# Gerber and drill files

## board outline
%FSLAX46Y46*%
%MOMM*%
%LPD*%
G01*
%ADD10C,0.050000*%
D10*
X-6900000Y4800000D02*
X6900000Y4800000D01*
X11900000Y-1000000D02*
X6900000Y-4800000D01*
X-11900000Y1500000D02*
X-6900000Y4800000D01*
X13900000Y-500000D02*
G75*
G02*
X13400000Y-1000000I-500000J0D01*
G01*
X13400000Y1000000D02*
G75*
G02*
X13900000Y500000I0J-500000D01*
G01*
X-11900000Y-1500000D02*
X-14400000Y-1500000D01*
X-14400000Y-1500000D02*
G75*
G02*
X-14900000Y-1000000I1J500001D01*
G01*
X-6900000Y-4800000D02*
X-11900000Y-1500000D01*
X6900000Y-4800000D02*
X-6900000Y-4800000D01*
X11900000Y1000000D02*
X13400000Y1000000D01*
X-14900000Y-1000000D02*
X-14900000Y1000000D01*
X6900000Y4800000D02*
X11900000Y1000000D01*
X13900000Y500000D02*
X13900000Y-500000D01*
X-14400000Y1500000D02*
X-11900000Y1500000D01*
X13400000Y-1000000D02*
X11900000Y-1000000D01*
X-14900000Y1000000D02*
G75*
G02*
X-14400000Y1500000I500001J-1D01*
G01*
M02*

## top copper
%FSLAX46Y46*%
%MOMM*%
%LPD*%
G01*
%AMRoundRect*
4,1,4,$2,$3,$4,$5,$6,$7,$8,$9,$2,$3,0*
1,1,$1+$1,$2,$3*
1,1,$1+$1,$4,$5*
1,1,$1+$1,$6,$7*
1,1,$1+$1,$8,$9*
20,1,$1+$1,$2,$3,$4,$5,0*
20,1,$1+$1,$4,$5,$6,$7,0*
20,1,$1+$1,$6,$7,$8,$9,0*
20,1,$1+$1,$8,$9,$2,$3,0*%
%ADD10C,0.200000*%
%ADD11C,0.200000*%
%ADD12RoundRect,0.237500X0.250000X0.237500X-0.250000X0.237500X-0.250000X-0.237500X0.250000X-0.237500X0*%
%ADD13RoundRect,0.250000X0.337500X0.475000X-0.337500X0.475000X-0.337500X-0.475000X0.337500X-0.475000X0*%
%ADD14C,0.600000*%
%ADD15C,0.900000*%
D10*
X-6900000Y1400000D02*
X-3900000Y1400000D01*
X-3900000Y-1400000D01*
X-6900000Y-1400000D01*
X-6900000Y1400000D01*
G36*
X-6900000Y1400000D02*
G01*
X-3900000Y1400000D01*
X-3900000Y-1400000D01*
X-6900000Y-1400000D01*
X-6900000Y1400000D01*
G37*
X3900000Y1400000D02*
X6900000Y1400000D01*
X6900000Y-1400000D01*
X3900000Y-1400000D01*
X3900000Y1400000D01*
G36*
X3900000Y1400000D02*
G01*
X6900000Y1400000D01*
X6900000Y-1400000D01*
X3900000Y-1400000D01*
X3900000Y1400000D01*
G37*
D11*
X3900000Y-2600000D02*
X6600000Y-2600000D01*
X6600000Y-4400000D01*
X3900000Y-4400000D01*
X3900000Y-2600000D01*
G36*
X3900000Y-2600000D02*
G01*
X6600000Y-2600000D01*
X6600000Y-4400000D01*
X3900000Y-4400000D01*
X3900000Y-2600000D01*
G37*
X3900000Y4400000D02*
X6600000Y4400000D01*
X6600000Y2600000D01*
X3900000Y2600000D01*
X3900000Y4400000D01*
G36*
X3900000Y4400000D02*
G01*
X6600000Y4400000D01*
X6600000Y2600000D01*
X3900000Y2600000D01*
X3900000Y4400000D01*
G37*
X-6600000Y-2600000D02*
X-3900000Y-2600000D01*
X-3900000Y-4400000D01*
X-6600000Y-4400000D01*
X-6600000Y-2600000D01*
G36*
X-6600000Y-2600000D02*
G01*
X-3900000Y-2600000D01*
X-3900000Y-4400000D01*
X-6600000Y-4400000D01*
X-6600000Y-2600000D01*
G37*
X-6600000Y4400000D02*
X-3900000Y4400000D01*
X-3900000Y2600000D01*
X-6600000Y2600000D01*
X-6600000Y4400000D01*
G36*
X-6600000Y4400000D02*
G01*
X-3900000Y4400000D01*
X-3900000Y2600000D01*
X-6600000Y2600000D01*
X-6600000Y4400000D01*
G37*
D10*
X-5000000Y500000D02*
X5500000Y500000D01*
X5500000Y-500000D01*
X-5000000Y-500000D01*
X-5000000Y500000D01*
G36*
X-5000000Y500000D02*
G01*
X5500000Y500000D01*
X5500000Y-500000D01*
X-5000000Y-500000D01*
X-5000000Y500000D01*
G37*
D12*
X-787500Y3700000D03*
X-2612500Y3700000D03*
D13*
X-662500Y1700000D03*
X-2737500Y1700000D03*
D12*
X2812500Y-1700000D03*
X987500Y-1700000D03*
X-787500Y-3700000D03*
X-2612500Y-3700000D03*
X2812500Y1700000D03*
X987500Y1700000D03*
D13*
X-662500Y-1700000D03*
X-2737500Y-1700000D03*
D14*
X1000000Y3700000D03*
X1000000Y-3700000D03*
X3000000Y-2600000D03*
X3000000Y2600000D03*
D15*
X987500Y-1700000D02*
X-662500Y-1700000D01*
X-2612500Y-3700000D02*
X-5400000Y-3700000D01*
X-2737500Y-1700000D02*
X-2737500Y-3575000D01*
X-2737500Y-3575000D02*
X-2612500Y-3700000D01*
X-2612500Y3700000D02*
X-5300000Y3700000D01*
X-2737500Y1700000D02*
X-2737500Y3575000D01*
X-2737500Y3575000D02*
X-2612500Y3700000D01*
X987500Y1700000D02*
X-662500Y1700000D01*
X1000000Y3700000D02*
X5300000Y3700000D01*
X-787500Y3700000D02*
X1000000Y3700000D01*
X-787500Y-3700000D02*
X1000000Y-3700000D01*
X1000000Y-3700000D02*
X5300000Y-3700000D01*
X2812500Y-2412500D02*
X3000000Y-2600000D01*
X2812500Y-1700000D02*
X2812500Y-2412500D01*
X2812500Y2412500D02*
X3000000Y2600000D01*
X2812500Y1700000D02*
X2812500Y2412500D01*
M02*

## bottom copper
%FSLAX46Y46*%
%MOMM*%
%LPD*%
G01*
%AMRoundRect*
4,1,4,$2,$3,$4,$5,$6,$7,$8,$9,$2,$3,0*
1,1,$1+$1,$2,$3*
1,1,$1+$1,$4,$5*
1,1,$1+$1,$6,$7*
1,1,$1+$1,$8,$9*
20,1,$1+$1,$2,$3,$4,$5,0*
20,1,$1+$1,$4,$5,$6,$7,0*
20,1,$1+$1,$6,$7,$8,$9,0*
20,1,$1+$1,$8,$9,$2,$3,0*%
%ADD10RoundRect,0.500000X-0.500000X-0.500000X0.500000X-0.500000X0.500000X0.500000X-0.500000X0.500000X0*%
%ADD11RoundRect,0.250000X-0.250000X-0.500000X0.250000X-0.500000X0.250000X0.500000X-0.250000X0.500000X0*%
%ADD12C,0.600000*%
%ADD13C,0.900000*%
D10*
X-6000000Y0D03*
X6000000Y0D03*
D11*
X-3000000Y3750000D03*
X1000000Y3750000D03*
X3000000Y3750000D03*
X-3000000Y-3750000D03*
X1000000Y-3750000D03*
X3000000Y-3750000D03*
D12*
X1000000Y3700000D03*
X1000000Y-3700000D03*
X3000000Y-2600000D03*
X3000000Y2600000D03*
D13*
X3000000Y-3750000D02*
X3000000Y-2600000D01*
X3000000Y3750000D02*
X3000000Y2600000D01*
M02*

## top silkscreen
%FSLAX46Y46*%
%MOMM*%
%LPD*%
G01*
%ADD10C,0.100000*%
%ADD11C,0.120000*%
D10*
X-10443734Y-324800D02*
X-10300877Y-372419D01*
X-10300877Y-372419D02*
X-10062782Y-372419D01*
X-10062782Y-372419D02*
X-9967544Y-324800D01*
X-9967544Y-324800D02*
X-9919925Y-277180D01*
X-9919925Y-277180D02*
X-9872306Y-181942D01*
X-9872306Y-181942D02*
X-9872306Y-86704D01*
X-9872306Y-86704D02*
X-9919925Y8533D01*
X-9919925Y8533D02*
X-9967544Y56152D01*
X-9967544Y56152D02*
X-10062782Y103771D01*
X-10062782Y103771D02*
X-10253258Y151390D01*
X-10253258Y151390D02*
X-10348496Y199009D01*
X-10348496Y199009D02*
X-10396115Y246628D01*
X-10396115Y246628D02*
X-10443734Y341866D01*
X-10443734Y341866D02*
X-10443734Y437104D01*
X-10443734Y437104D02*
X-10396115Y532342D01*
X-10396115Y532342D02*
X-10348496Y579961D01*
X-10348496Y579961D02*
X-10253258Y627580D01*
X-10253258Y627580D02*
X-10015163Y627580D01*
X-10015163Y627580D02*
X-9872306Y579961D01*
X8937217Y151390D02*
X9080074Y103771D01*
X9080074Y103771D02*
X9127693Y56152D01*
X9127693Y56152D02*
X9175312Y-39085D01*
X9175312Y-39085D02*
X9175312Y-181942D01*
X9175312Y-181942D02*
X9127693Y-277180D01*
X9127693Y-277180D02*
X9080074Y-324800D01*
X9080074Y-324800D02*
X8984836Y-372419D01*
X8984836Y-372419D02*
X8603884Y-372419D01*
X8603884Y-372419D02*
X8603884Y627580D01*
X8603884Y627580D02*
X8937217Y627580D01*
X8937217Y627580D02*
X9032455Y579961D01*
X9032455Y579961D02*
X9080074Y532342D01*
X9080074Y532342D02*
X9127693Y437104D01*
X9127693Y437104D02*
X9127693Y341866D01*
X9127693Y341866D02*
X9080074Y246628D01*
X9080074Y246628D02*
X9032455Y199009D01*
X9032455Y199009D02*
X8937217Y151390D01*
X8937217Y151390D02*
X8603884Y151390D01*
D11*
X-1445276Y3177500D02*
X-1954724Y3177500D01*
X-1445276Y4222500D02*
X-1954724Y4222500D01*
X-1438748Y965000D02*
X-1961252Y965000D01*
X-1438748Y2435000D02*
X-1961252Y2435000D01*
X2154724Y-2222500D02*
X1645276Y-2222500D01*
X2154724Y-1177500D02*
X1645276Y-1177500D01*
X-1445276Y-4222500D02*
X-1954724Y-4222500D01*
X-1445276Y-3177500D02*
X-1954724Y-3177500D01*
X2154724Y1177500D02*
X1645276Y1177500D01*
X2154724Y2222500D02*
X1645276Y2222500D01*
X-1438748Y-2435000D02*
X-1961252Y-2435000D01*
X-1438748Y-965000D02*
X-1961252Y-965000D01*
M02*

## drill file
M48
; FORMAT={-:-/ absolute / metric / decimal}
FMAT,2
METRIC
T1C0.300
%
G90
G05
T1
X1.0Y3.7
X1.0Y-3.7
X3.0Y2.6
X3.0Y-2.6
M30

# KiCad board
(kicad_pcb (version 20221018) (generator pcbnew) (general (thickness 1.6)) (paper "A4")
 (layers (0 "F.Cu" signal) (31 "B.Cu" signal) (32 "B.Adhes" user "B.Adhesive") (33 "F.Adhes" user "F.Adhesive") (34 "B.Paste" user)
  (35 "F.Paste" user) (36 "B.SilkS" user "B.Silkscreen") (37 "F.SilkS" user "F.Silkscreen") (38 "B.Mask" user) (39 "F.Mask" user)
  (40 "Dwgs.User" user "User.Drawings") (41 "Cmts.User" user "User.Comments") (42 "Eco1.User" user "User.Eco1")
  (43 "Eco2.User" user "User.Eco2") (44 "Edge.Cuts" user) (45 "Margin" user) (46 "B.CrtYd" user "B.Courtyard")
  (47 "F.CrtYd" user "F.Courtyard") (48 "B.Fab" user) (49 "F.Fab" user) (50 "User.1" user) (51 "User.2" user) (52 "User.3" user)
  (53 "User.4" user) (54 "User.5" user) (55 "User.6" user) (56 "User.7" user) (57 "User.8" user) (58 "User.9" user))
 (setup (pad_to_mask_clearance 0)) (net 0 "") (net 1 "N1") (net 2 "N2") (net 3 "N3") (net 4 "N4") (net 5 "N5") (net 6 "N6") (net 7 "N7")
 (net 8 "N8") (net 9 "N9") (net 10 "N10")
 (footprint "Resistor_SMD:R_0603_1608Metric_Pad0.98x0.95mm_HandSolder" (layer "F.Cu") (at -1.7 -3.7 180)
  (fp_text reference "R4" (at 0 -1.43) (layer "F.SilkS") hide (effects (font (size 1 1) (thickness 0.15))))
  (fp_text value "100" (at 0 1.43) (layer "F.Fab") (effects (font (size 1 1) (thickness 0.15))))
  (fp_line (start -0.254724 -0.5225) (end 0.254724 -0.5225) (stroke (width 0.12) (type solid)) (layer "F.SilkS"))
  (fp_line (start -0.254724 0.5225) (end 0.254724 0.5225) (stroke (width 0.12) (type solid)) (layer "F.SilkS"))
  (pad "1" smd roundrect (at -0.9125 0 180) (size 0.975 0.95) (layers "F.Cu" "F.Paste" "F.Mask") (roundrect_rratio 0.25) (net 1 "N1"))
  (pad "2" smd roundrect (at 0.9125 0 180) (size 0.975 0.95) (layers "F.Cu" "F.Paste" "F.Mask") (roundrect_rratio 0.25) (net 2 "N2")))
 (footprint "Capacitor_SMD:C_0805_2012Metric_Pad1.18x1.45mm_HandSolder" (layer "F.Cu") (at -1.7 -1.7 180)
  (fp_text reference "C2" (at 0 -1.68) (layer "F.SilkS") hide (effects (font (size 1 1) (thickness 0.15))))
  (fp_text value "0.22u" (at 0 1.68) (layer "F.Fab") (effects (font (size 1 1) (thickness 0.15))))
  (fp_line (start -0.261252 -0.735) (end 0.261252 -0.735) (stroke (width 0.12) (type solid)) (layer "F.SilkS"))
  (fp_line (start -0.261252 0.735) (end 0.261252 0.735) (stroke (width 0.12) (type solid)) (layer "F.SilkS"))
  (pad "1" smd roundrect (at -1.0375 0 180) (size 1.175 1.45) (layers "F.Cu" "F.Paste" "F.Mask") (roundrect_rratio 0.2127659574)
   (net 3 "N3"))
  (pad "2" smd roundrect (at 1.0375 0 180) (size 1.175 1.45) (layers "F.Cu" "F.Paste" "F.Mask") (roundrect_rratio 0.2127659574) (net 2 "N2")))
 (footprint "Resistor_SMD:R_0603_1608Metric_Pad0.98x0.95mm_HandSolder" (layer "F.Cu") (at 1.9 1.7 180)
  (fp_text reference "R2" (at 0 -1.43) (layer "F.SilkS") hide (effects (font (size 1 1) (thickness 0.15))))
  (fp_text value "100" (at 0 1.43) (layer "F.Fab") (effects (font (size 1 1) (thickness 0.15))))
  (fp_line (start -0.254724 -0.5225) (end 0.254724 -0.5225) (stroke (width 0.12) (type solid)) (layer "F.SilkS"))
  (fp_line (start -0.254724 0.5225) (end 0.254724 0.5225) (stroke (width 0.12) (type solid)) (layer "F.SilkS"))
  (pad "1" smd roundrect (at -0.9125 0 180) (size 0.975 0.95) (layers "F.Cu" "F.Paste" "F.Mask") (roundrect_rratio 0.25) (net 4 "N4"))
  (pad "2" smd roundrect (at 0.9125 0 180) (size 0.975 0.95) (layers "F.Cu" "F.Paste" "F.Mask") (roundrect_rratio 0.25) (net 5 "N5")))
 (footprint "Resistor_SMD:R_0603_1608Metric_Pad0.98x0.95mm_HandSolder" (layer "F.Cu") (at -1.7 3.7 180)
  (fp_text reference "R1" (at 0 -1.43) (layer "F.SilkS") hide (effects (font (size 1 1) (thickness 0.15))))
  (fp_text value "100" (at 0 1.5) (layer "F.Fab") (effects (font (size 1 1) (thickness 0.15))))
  (fp_line (start -0.254724 -0.5225) (end 0.254724 -0.5225) (stroke (width 0.12) (type solid)) (layer "F.SilkS"))
  (fp_line (start -0.254724 0.5225) (end 0.254724 0.5225) (stroke (width 0.12) (type solid)) (layer "F.SilkS"))
  (pad "1" smd roundrect (at -0.9125 0 180) (size 0.975 0.95) (layers "F.Cu" "F.Paste" "F.Mask") (roundrect_rratio 0.25) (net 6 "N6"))
  (pad "2" smd roundrect (at 0.9125 0 180) (size 0.975 0.95) (layers "F.Cu" "F.Paste" "F.Mask") (roundrect_rratio 0.25) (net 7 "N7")))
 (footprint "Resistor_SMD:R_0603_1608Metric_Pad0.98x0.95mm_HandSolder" (layer "F.Cu") (at 1.9 -1.7 180)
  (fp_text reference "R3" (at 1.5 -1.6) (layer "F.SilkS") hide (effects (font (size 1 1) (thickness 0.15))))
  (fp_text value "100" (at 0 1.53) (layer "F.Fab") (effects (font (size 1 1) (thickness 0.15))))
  (fp_line (start -0.254724 -0.5225) (end 0.254724 -0.5225) (stroke (width 0.12) (type solid)) (layer "F.SilkS"))
  (fp_line (start -0.254724 0.5225) (end 0.254724 0.5225) (stroke (width 0.12) (type solid)) (layer "F.SilkS"))
  (pad "1" smd roundrect (at -0.9125 0 180) (size 0.975 0.95) (layers "F.Cu" "F.Paste" "F.Mask") (roundrect_rratio 0.25) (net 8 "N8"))
  (pad "2" smd roundrect (at 0.9125 0 180) (size 0.975 0.95) (layers "F.Cu" "F.Paste" "F.Mask") (roundrect_rratio 0.25) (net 3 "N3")))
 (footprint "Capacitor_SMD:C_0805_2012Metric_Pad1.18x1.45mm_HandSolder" (layer "F.Cu") (at -1.7 1.7 180)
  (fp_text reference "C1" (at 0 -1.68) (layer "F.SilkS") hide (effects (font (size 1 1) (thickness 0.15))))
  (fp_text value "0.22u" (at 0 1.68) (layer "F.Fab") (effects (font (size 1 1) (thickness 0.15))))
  (fp_line (start -0.261252 -0.735) (end 0.261252 -0.735) (stroke (width 0.12) (type solid)) (layer "F.SilkS"))
  (fp_line (start -0.261252 0.735) (end 0.261252 0.735) (stroke (width 0.12) (type solid)) (layer "F.SilkS"))
  (pad "1" smd roundrect (at -1.0375 0 180) (size 1.175 1.45) (layers "F.Cu" "F.Paste" "F.Mask") (roundrect_rratio 0.2127659574)
   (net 5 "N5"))
  (pad "2" smd roundrect (at 1.0375 0 180) (size 1.175 1.45) (layers "F.Cu" "F.Paste" "F.Mask") (roundrect_rratio 0.2127659574) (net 7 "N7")))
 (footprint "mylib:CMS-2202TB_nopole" (layer "B.Cu") (at 0 0)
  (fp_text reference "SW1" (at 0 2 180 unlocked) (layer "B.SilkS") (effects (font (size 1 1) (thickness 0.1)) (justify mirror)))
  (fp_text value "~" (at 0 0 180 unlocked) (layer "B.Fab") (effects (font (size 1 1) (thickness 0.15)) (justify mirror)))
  (pad "" smd roundrect (at -6 0) (size 2 2) (layers "B.Cu" "B.Paste" "B.Mask") (roundrect_rratio 0.25) (thermal_bridge_angle 45))
  (pad "" smd roundrect (at 6 0) (size 2 2) (layers "B.Cu" "B.Paste" "B.Mask") (roundrect_rratio 0.25) (thermal_bridge_angle 45))
  (pad "1" smd roundrect (at -3 -3.75) (size 1 1.5) (layers "B.Cu" "B.Paste" "B.Mask") (roundrect_rratio 0.25) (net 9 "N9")
   (thermal_bridge_angle 45))
  (pad "2" smd roundrect (at 1 -3.75) (size 1 1.5) (layers "B.Cu" "B.Paste" "B.Mask") (roundrect_rratio 0.25) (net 1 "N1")
   (thermal_bridge_angle 45))
  (pad "3" smd roundrect (at 3 -3.75) (size 1 1.5) (layers "B.Cu" "B.Paste" "B.Mask") (roundrect_rratio 0.25) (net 8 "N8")
   (thermal_bridge_angle 45))
  (pad "4" smd roundrect (at -3 3.75) (size 1 1.5) (layers "B.Cu" "B.Paste" "B.Mask") (roundrect_rratio 0.25) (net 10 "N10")
   (thermal_bridge_angle 45))
  (pad "5" smd roundrect (at 1 3.75) (size 1 1.5) (layers "B.Cu" "B.Paste" "B.Mask") (roundrect_rratio 0.25) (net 6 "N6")
   (thermal_bridge_angle 45))
  (pad "6" smd roundrect (at 3 3.75) (size 1 1.5) (layers "B.Cu" "B.Paste" "B.Mask") (roundrect_rratio 0.25) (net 4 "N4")
   (thermal_bridge_angle 45)))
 (gr_rect (start -6.9 -1.4) (end -3.9 1.4) (stroke (width 0.2) (type solid)) (fill solid) (layer "F.Cu"))
 (gr_rect (start 3.9 -1.4) (end 6.9 1.4) (stroke (width 0.2) (type solid)) (fill solid) (layer "F.Cu"))
 (gr_rect (start 3.9 2.6) (end 6.6 4.4) (stroke (width 0.2) (type solid)) (fill solid) (layer "F.Cu"))
 (gr_rect (start 3.9 -4.4) (end 6.6 -2.6) (stroke (width 0.2) (type solid)) (fill solid) (layer "F.Cu"))
 (gr_rect (start -6.6 2.6) (end -3.9 4.4) (stroke (width 0.2) (type solid)) (fill solid) (layer "F.Cu"))
 (gr_rect (start -6.6 -4.4) (end -3.9 -2.6) (stroke (width 0.2) (type solid)) (fill solid) (layer "F.Cu"))
 (gr_rect (start -5 -0.5) (end 5.5 0.5) (stroke (width 0.2) (type solid)) (fill solid) (layer "F.Cu"))
 (gr_line (start -6.9 -4.8) (end 6.9 -4.8) (stroke (width 0.05) (type default)) (layer "Edge.Cuts"))
 (gr_line (start 11.9 1) (end 6.9 4.8) (stroke (width 0.05) (type default)) (layer "Edge.Cuts"))
 (gr_line (start -11.9 -1.5) (end -6.9 -4.8) (stroke (width 0.05) (type default)) (layer "Edge.Cuts"))
 (gr_arc (start 13.9 0.5) (mid 13.753553 0.853553) (end 13.4 1) (stroke (width 0.05) (type default)) (layer "Edge.Cuts"))
 (gr_arc (start 13.4 -1) (mid 13.753553 -0.853553) (end 13.9 -0.5) (stroke (width 0.05) (type default)) (layer "Edge.Cuts"))
 (gr_line (start -11.9 1.5) (end -14.4 1.5) (stroke (width 0.05) (type default)) (layer "Edge.Cuts"))
 (gr_arc (start -14.4 1.5) (mid -14.753553 1.353553) (end -14.9 1) (stroke (width 0.05) (type default)) (layer "Edge.Cuts"))
 (gr_line (start -6.9 4.8) (end -11.9 1.5) (stroke (width 0.05) (type default)) (layer "Edge.Cuts"))
 (gr_line (start 6.9 4.8) (end -6.9 4.8) (stroke (width 0.05) (type default)) (layer "Edge.Cuts"))
 (gr_line (start 11.9 -1) (end 13.4 -1) (stroke (width 0.05) (type default)) (layer "Edge.Cuts"))
 (gr_line (start -14.9 1) (end -14.9 -1) (stroke (width 0.05) (type default)) (layer "Edge.Cuts"))
 (gr_line (start 6.9 -4.8) (end 11.9 -1) (stroke (width 0.05) (type default)) (layer "Edge.Cuts"))
 (gr_line (start 13.9 -0.5) (end 13.9 0.5) (stroke (width 0.05) (type default)) (layer "Edge.Cuts"))
 (gr_line (start -14.4 -1.5) (end -11.9 -1.5) (stroke (width 0.05) (type default)) (layer "Edge.Cuts"))
 (gr_line (start 13.4 1) (end 11.9 1) (stroke (width 0.05) (type default)) (layer "Edge.Cuts"))
 (gr_arc (start -14.9 -1) (mid -14.753553 -1.353553) (end -14.4 -1.5) (stroke (width 0.05) (type default)) (layer "Edge.Cuts"))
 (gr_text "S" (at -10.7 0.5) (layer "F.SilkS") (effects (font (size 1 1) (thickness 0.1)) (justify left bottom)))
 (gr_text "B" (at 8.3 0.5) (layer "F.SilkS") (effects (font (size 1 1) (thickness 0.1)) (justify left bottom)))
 (segment (start 0.9875 1.7) (end -0.6625 1.7) (width 0.9) (layer "F.Cu") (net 5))
 (segment (start -2.6125 3.7) (end -5.4 3.7) (width 0.9) (layer "F.Cu") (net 7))
 (segment (start -2.7375 1.7) (end -2.7375 3.575) (width 0.9) (layer "F.Cu") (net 7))
 (segment (start -2.7375 3.575) (end -2.6125 3.7) (width 0.9) (layer "F.Cu") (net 7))
 (segment (start -2.6125 -3.7) (end -5.3 -3.7) (width 0.9) (layer "F.Cu") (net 2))
 (segment (start -2.7375 -1.7) (end -2.7375 -3.575) (width 0.9) (layer "F.Cu") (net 2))
 (segment (start -2.7375 -3.575) (end -2.6125 -3.7) (width 0.9) (layer "F.Cu") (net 2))
 (segment (start 0.9875 -1.7) (end -0.6625 -1.7) (width 0.9) (layer "F.Cu") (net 3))
 (segment (start 1 -3.7) (end 5.3 -3.7) (width 0.9) (layer "F.Cu") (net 1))
 (segment (start -0.7875 -3.7) (end 1 -3.7) (width 0.9) (layer "F.Cu") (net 1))
 (via (at 1 -3.7) (size 0.6) (drill 0.3) (layers "F.Cu" "B.Cu") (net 1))
 (segment (start -0.7875 3.7) (end 1 3.7) (width 0.9) (layer "F.Cu") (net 6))
 (segment (start 1 3.7) (end 5.3 3.7) (width 0.9) (layer "F.Cu") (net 6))
 (via (at 1 3.7) (size 0.6) (drill 0.3) (layers "F.Cu" "B.Cu") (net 6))
 (segment (start 2.8125 2.4125) (end 3 2.6) (width 0.9) (layer "F.Cu") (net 4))
 (segment (start 2.8125 1.7) (end 2.8125 2.4125) (width 0.9) (layer "F.Cu") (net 4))
 (via (at 3 2.6) (size 0.6) (drill 0.3) (layers "F.Cu" "B.Cu") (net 4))
 (segment (start 3 3.75) (end 3 2.6) (width 0.9) (layer "B.Cu") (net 4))
 (segment (start 2.8125 -2.4125) (end 3 -2.6) (width 0.9) (layer "F.Cu") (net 8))
 (segment (start 2.8125 -1.7) (end 2.8125 -2.4125) (width 0.9) (layer "F.Cu") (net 8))
 (via (at 3 -2.6) (size 0.6) (drill 0.3) (layers "F.Cu" "B.Cu") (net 8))
 (segment (start 3 -3.75) (end 3 -2.6) (width 0.9) (layer "B.Cu") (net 8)))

